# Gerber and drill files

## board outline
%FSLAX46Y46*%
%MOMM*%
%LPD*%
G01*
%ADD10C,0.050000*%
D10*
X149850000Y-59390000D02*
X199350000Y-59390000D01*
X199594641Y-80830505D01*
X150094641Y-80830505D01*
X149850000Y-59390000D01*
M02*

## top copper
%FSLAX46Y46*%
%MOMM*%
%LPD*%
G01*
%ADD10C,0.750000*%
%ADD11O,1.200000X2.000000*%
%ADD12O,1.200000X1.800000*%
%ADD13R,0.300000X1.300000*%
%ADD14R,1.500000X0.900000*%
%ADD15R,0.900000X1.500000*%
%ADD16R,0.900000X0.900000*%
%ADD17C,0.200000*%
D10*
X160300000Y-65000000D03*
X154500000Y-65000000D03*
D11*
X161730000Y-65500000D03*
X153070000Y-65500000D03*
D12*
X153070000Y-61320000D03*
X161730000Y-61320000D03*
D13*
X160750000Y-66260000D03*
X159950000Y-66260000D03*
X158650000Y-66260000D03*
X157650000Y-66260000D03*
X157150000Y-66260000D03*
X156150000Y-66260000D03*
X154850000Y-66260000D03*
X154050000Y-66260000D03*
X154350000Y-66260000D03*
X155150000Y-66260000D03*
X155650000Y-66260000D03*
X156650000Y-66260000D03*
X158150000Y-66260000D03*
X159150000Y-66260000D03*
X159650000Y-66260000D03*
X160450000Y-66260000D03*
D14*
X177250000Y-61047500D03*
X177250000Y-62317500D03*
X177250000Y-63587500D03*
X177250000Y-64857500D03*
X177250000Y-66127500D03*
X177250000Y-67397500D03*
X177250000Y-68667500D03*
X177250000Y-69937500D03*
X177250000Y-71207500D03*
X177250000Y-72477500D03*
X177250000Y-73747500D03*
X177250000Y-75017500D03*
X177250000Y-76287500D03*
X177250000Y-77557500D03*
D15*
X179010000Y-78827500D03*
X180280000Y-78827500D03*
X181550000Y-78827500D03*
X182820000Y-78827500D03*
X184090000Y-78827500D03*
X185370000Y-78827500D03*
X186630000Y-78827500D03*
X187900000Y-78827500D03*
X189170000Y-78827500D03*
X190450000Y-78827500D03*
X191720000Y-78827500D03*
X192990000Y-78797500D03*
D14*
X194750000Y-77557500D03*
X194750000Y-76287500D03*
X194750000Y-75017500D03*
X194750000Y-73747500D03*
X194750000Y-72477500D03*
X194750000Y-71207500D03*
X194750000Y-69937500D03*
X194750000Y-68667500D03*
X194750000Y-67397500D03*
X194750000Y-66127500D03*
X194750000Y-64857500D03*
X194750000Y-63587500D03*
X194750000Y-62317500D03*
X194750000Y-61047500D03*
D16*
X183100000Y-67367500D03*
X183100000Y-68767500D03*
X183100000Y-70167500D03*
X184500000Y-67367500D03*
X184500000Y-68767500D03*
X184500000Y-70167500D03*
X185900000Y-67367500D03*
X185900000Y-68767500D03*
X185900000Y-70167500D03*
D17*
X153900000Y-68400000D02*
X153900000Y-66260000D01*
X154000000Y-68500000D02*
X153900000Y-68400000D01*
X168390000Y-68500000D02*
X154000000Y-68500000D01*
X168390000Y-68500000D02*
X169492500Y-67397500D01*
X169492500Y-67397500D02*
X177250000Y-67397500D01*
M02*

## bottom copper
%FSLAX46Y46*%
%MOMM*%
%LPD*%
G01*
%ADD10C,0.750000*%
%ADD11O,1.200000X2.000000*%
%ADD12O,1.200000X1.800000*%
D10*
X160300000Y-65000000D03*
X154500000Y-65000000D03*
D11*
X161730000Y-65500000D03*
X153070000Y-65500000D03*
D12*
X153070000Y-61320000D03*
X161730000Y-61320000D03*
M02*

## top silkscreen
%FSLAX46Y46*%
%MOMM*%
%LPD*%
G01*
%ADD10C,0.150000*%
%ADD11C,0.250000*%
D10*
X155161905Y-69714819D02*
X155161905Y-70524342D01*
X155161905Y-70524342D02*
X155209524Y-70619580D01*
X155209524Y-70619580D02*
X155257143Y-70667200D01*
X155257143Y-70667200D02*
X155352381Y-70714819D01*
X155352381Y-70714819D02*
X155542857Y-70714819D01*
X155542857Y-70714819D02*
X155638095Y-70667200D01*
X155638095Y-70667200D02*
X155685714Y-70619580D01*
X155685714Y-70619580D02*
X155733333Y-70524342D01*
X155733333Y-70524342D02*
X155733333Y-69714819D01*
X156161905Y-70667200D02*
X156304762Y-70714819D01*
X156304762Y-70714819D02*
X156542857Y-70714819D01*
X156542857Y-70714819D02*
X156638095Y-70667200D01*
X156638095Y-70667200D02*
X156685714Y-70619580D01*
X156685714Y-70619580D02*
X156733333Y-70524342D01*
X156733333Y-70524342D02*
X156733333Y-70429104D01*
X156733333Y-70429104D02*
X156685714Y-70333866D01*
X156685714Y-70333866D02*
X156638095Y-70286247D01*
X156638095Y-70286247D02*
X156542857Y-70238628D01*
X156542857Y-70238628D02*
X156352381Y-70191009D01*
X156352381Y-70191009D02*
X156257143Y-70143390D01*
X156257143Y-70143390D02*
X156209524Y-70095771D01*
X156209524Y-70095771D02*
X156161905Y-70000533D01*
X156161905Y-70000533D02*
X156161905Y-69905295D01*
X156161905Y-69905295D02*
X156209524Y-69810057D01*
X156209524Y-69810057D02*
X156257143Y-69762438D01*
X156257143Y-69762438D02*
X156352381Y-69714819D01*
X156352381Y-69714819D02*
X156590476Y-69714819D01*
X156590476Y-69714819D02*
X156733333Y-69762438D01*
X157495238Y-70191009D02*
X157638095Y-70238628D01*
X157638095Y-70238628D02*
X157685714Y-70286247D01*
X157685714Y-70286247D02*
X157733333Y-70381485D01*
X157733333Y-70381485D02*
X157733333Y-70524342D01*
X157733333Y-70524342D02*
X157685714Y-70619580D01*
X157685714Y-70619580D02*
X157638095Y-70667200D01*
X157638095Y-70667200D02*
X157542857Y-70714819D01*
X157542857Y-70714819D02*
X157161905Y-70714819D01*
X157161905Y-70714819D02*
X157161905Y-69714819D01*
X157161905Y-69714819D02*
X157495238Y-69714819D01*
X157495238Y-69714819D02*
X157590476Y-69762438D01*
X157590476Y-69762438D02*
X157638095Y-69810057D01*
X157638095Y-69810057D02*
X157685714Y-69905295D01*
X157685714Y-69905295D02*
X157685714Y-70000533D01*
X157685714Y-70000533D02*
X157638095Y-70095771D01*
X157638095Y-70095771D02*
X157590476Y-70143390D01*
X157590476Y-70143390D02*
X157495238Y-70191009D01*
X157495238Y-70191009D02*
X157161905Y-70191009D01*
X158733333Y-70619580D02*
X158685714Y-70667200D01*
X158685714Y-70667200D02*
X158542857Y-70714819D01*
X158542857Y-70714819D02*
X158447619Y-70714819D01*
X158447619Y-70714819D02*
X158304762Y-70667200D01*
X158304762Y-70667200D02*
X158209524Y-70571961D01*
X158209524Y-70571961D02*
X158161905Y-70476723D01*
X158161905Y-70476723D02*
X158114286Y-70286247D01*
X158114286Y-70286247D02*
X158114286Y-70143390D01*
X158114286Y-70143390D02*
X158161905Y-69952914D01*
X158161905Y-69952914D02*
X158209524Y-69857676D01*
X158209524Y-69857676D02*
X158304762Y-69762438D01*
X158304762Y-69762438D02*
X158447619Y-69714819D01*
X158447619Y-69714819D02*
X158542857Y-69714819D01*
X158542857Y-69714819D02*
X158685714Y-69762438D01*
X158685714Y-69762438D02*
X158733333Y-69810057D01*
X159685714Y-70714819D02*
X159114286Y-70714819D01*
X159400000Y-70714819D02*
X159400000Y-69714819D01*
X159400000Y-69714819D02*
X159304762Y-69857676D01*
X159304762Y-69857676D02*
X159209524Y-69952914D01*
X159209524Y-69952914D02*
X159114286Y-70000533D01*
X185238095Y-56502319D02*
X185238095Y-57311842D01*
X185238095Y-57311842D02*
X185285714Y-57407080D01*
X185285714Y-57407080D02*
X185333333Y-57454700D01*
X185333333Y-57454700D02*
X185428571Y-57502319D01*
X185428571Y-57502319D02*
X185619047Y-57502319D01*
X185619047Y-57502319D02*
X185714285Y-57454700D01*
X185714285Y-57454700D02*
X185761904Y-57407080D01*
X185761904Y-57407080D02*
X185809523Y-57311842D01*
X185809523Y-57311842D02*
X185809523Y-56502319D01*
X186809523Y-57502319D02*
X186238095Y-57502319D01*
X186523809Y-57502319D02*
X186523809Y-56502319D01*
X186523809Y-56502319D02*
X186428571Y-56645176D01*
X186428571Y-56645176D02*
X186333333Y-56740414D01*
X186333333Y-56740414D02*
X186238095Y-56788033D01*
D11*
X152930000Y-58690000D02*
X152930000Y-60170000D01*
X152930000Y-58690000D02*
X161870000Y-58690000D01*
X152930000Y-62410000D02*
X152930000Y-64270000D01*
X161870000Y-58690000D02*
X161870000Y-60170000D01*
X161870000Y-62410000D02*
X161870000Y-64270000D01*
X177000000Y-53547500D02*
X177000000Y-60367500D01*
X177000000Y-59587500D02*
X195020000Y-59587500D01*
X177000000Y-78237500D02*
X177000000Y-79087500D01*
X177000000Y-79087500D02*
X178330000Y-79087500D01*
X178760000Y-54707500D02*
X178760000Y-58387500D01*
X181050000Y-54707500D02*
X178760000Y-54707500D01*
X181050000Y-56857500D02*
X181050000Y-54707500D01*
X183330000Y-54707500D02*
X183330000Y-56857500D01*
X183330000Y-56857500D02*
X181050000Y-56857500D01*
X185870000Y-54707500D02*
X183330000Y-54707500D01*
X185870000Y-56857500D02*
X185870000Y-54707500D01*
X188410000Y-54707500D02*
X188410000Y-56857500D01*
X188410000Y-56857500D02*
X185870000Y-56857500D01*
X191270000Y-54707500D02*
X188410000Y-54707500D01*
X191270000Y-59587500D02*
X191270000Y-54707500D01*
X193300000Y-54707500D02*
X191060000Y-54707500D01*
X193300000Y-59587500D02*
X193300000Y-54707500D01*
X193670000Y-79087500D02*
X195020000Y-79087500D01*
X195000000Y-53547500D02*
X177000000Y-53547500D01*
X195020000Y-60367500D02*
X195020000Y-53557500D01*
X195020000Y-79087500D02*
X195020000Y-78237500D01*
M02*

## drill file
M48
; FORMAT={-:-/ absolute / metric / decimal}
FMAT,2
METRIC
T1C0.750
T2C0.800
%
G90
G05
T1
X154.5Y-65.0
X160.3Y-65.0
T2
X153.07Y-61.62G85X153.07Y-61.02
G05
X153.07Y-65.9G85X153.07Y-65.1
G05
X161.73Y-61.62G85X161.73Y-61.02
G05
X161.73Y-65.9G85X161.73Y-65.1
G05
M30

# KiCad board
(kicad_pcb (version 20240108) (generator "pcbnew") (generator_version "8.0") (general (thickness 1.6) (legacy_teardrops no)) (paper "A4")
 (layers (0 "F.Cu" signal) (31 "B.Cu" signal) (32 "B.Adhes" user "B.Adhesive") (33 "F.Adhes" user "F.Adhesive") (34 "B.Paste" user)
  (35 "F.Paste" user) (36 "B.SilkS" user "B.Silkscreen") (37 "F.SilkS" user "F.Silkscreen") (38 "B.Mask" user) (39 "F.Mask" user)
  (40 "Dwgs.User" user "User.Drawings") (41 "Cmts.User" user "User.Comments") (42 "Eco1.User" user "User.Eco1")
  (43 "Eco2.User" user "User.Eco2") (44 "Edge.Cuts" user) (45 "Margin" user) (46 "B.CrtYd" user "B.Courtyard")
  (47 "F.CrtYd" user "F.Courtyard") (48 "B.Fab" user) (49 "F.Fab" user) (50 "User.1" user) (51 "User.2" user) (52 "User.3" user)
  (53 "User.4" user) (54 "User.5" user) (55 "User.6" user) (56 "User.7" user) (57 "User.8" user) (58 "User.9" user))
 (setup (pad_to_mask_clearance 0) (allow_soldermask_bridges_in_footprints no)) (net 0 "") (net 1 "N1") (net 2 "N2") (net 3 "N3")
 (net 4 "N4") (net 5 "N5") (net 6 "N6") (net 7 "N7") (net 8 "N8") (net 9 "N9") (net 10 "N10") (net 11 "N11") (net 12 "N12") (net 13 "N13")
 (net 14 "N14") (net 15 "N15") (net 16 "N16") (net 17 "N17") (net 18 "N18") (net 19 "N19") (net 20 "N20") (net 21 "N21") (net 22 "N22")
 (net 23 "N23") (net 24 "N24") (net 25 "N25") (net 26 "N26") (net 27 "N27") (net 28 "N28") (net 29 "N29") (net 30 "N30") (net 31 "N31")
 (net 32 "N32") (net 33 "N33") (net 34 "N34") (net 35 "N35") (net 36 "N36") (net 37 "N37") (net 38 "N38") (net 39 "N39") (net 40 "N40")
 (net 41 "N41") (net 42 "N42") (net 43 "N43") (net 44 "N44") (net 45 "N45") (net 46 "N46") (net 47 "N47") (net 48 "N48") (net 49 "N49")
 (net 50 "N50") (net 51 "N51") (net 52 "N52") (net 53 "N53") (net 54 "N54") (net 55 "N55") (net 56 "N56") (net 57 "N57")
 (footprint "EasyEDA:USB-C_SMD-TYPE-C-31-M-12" (layer "F.Cu") (at 157.4 63.79 180)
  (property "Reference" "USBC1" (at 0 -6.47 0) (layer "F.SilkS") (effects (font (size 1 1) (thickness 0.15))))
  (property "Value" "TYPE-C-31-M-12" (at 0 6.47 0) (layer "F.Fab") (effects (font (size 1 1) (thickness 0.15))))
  (fp_line (start 4.47 5.1) (end 4.47 3.62) (stroke (width 0.25) (type solid)) (layer "F.SilkS"))
  (fp_line (start 4.47 5.1) (end -4.47 5.1) (stroke (width 0.25) (type solid)) (layer "F.SilkS"))
  (fp_line (start 4.47 1.38) (end 4.47 -0.48) (stroke (width 0.25) (type solid)) (layer "F.SilkS"))
  (fp_line (start -4.47 5.1) (end -4.47 3.62) (stroke (width 0.25) (type solid)) (layer "F.SilkS"))
  (fp_line (start -4.47 1.38) (end -4.47 -0.48) (stroke (width 0.25) (type solid)) (layer "F.SilkS"))
  (pad "" thru_hole circle (at -2.9 -1.21 180) (size 0.75 0.75) (drill 0.75) (layers "*.Cu" "*.Mask") (remove_unused_layers no))
  (pad "" thru_hole circle (at 2.9 -1.21 180) (size 0.75 0.75) (drill 0.75) (layers "*.Cu" "*.Mask") (remove_unused_layers no))
  (pad "0" thru_hole oval (at -4.33 -1.71 180) (size 1.2 2) (drill oval 0.799998 1.600022) (layers "*.Cu" "*.Mask")
   (remove_unused_layers no) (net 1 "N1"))
  (pad "1" thru_hole oval (at 4.33 -1.71 180) (size 1.2 2) (drill oval 0.799998 1.599971) (layers "*.Cu" "*.Mask") (remove_unused_layers no))
  (pad "2" thru_hole oval (at 4.33 2.47 180) (size 1.2 1.8) (drill oval 0.799998 1.399997) (layers "*.Cu" "*.Mask")
   (remove_unused_layers no))
  (pad "3" thru_hole oval (at -4.33 2.47 180) (size 1.2 1.8) (drill oval 0.799998 1.399997) (layers "*.Cu" "*.Mask")
   (remove_unused_layers no))
  (pad "A1" smd rect (at -3.35 -2.47 180) (size 0.3 1.3) (layers "F.Cu" "F.Paste" "F.Mask") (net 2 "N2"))
  (pad "A4" smd rect (at -2.55 -2.47 180) (size 0.3 1.3) (layers "F.Cu" "F.Paste" "F.Mask") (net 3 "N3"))
  (pad "A5" smd rect (at -1.25 -2.47 180) (size 0.3 1.3) (layers "F.Cu" "F.Paste" "F.Mask") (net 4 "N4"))
  (pad "A6" smd rect (at -0.25 -2.47 180) (size 0.3 1.3) (layers "F.Cu" "F.Paste" "F.Mask") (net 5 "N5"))
  (pad "A7" smd rect (at 0.25 -2.47 180) (size 0.3 1.3) (layers "F.Cu" "F.Paste" "F.Mask") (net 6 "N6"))
  (pad "A8" smd rect (at 1.25 -2.47 180) (size 0.3 1.3) (layers "F.Cu" "F.Paste" "F.Mask") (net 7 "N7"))
  (pad "A9" smd rect (at 2.55 -2.47 180) (size 0.3 1.3) (layers "F.Cu" "F.Paste" "F.Mask") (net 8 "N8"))
  (pad "A12" smd rect (at 3.35 -2.47 180) (size 0.3 1.3) (layers "F.Cu" "F.Paste" "F.Mask") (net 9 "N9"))
  (pad "B1" smd rect (at 3.05 -2.47 180) (size 0.3 1.3) (layers "F.Cu" "F.Paste" "F.Mask") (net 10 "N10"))
  (pad "B4" smd rect (at 2.25 -2.47 180) (size 0.3 1.3) (layers "F.Cu" "F.Paste" "F.Mask") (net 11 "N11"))
  (pad "B5" smd rect (at 1.75 -2.47 180) (size 0.3 1.3) (layers "F.Cu" "F.Paste" "F.Mask") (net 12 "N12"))
  (pad "B6" smd rect (at 0.75 -2.47 180) (size 0.3 1.3) (layers "F.Cu" "F.Paste" "F.Mask") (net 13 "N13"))
  (pad "B7" smd rect (at -0.75 -2.47 180) (size 0.3 1.3) (layers "F.Cu" "F.Paste" "F.Mask") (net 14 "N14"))
  (pad "B8" smd rect (at -1.75 -2.47 180) (size 0.3 1.3) (layers "F.Cu" "F.Paste" "F.Mask") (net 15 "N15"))
  (pad "B9" smd rect (at -2.25 -2.47 180) (size 0.3 1.3) (layers "F.Cu" "F.Paste" "F.Mask") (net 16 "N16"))
  (pad "B12" smd rect (at -3.05 -2.47 180) (size 0.3 1.3) (layers "F.Cu" "F.Paste" "F.Mask") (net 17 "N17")))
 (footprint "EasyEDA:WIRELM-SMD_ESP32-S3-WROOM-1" (layer "F.Cu") (at 186 69.9375)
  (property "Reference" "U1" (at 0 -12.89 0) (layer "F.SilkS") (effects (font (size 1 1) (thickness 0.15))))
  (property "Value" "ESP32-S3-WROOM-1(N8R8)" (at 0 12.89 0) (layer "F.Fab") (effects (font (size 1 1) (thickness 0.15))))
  (fp_line (start -9 -16.39) (end -9 -9.57) (stroke (width 0.25) (type solid)) (layer "F.SilkS"))
  (fp_line (start -9 -10.35) (end 9.02 -10.35) (stroke (width 0.25) (type solid)) (layer "F.SilkS"))
  (fp_line (start -9 8.3) (end -9 9.15) (stroke (width 0.25) (type solid)) (layer "F.SilkS"))
  (fp_line (start -9 9.15) (end -7.67 9.15) (stroke (width 0.25) (type solid)) (layer "F.SilkS"))
  (fp_line (start -7.24 -15.23) (end -7.24 -11.55) (stroke (width 0.25) (type solid)) (layer "F.SilkS"))
  (fp_line (start -4.95 -15.23) (end -7.24 -15.23) (stroke (width 0.25) (type solid)) (layer "F.SilkS"))
  (fp_line (start -4.95 -13.08) (end -4.95 -15.23) (stroke (width 0.25) (type solid)) (layer "F.SilkS"))
  (fp_line (start -2.67 -15.23) (end -2.67 -13.08) (stroke (width 0.25) (type solid)) (layer "F.SilkS"))
  (fp_line (start -2.67 -13.08) (end -4.95 -13.08) (stroke (width 0.25) (type solid)) (layer "F.SilkS"))
  (fp_line (start -0.13 -15.23) (end -2.67 -15.23) (stroke (width 0.25) (type solid)) (layer "F.SilkS"))
  (fp_line (start -0.13 -13.08) (end -0.13 -15.23) (stroke (width 0.25) (type solid)) (layer "F.SilkS"))
  (fp_line (start 2.41 -15.23) (end 2.41 -13.08) (stroke (width 0.25) (type solid)) (layer "F.SilkS"))
  (fp_line (start 2.41 -13.08) (end -0.13 -13.08) (stroke (width 0.25) (type solid)) (layer "F.SilkS"))
  (fp_line (start 5.27 -15.23) (end 2.41 -15.23) (stroke (width 0.25) (type solid)) (layer "F.SilkS"))
  (fp_line (start 5.27 -10.35) (end 5.27 -15.23) (stroke (width 0.25) (type solid)) (layer "F.SilkS"))
  (fp_line (start 7.3 -15.23) (end 5.06 -15.23) (stroke (width 0.25) (type solid)) (layer "F.SilkS"))
  (fp_line (start 7.3 -10.35) (end 7.3 -15.23) (stroke (width 0.25) (type solid)) (layer "F.SilkS"))
  (fp_line (start 7.67 9.15) (end 9.02 9.15) (stroke (width 0.25) (type solid)) (layer "F.SilkS"))
  (fp_line (start 9 -16.39) (end -9 -16.39) (stroke (width 0.25) (type solid)) (layer "F.SilkS"))
  (fp_line (start 9.02 -9.57) (end 9.02 -16.38) (stroke (width 0.25) (type solid)) (layer "F.SilkS"))
  (fp_line (start 9.02 9.15) (end 9.02 8.3) (stroke (width 0.25) (type solid)) (layer "F.SilkS"))
  (pad "1" smd rect (at -8.75 -8.89) (size 1.5 0.9) (layers "F.Cu" "F.Paste" "F.Mask") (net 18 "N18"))
  (pad "2" smd rect (at -8.75 -7.62) (size 1.5 0.9) (layers "F.Cu" "F.Paste" "F.Mask") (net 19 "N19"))
  (pad "3" smd rect (at -8.75 -6.35) (size 1.5 0.9) (layers "F.Cu" "F.Paste" "F.Mask") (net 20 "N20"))
  (pad "4" smd rect (at -8.75 -5.08) (size 1.5 0.9) (layers "F.Cu" "F.Paste" "F.Mask") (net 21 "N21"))
  (pad "5" smd rect (at -8.75 -3.81) (size 1.5 0.9) (layers "F.Cu" "F.Paste" "F.Mask") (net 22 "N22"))
  (pad "6" smd rect (at -8.75 -2.54) (size 1.5 0.9) (layers "F.Cu" "F.Paste" "F.Mask") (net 9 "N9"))
  (pad "7" smd rect (at -8.75 -1.27) (size 1.5 0.9) (layers "F.Cu" "F.Paste" "F.Mask") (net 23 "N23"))
  (pad "8" smd rect (at -8.75 0) (size 1.5 0.9) (layers "F.Cu" "F.Paste" "F.Mask") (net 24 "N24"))
  (pad "9" smd rect (at -8.75 1.27) (size 1.5 0.9) (layers "F.Cu" "F.Paste" "F.Mask") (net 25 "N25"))
  (pad "10" smd rect (at -8.75 2.54) (size 1.5 0.9) (layers "F.Cu" "F.Paste" "F.Mask") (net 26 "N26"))
  (pad "11" smd rect (at -8.75 3.81) (size 1.5 0.9) (layers "F.Cu" "F.Paste" "F.Mask") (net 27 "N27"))
  (pad "12" smd rect (at -8.75 5.08) (size 1.5 0.9) (layers "F.Cu" "F.Paste" "F.Mask") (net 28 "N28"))
  (pad "13" smd rect (at -8.75 6.35) (size 1.5 0.9) (layers "F.Cu" "F.Paste" "F.Mask") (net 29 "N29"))
  (pad "14" smd rect (at -8.75 7.62) (size 1.5 0.9) (layers "F.Cu" "F.Paste" "F.Mask") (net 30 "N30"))
  (pad "15" smd rect (at -6.99 8.89 90) (size 1.5 0.9) (layers "F.Cu" "F.Paste" "F.Mask") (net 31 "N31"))
  (pad "16" smd rect (at -5.72 8.89 90) (size 1.5 0.9) (layers "F.Cu" "F.Paste" "F.Mask") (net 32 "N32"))
  (pad "17" smd rect (at -4.45 8.89 90) (size 1.5 0.9) (layers "F.Cu" "F.Paste" "F.Mask") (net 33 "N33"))
  (pad "18" smd rect (at -3.18 8.89 90) (size 1.5 0.9) (layers "F.Cu" "F.Paste" "F.Mask") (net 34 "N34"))
  (pad "19" smd rect (at -1.91 8.89 90) (size 1.5 0.9) (layers "F.Cu" "F.Paste" "F.Mask") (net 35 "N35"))
  (pad "20" smd rect (at -0.63 8.89 90) (size 1.5 0.9) (layers "F.Cu" "F.Paste" "F.Mask") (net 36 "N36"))
  (pad "21" smd rect (at 0.63 8.89 90) (size 1.5 0.9) (layers "F.Cu" "F.Paste" "F.Mask") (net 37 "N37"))
  (pad "22" smd rect (at 1.9 8.89 90) (size 1.5 0.9) (layers "F.Cu" "F.Paste" "F.Mask") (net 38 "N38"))
  (pad "23" smd rect (at 3.17 8.89 90) (size 1.5 0.9) (layers "F.Cu" "F.Paste" "F.Mask") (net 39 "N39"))
  (pad "24" smd rect (at 4.45 8.89 90) (size 1.5 0.9) (layers "F.Cu" "F.Paste" "F.Mask") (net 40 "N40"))
  (pad "25" smd rect (at 5.72 8.89 90) (size 1.5 0.9) (layers "F.Cu" "F.Paste" "F.Mask") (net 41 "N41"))
  (pad "26" smd rect (at 6.99 8.86 90) (size 1.5 0.9) (layers "F.Cu" "F.Paste" "F.Mask") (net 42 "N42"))
  (pad "27" smd rect (at 8.75 7.62 180) (size 1.5 0.9) (layers "F.Cu" "F.Paste" "F.Mask") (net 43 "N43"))
  (pad "28" smd rect (at 8.75 6.35 180) (size 1.5 0.9) (layers "F.Cu" "F.Paste" "F.Mask") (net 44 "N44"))
  (pad "29" smd rect (at 8.75 5.08 180) (size 1.5 0.9) (layers "F.Cu" "F.Paste" "F.Mask") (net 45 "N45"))
  (pad "30" smd rect (at 8.75 3.81 180) (size 1.5 0.9) (layers "F.Cu" "F.Paste" "F.Mask") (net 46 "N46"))
  (pad "31" smd rect (at 8.75 2.54 180) (size 1.5 0.9) (layers "F.Cu" "F.Paste" "F.Mask") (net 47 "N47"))
  (pad "32" smd rect (at 8.75 1.27 180) (size 1.5 0.9) (layers "F.Cu" "F.Paste" "F.Mask") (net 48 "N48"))
  (pad "33" smd rect (at 8.75 0 180) (size 1.5 0.9) (layers "F.Cu" "F.Paste" "F.Mask") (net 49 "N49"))
  (pad "34" smd rect (at 8.75 -1.27 180) (size 1.5 0.9) (layers "F.Cu" "F.Paste" "F.Mask") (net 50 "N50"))
  (pad "35" smd rect (at 8.75 -2.54 180) (size 1.5 0.9) (layers "F.Cu" "F.Paste" "F.Mask") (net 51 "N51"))
  (pad "36" smd rect (at 8.75 -3.81 180) (size 1.5 0.9) (layers "F.Cu" "F.Paste" "F.Mask") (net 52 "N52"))
  (pad "37" smd rect (at 8.75 -5.08 180) (size 1.5 0.9) (layers "F.Cu" "F.Paste" "F.Mask") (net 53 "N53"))
  (pad "38" smd rect (at 8.75 -6.35 180) (size 1.5 0.9) (layers "F.Cu" "F.Paste" "F.Mask") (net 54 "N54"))
  (pad "39" smd rect (at 8.75 -7.62 180) (size 1.5 0.9) (layers "F.Cu" "F.Paste" "F.Mask") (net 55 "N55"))
  (pad "40" smd rect (at 8.75 -8.89 180) (size 1.5 0.9) (layers "F.Cu" "F.Paste" "F.Mask") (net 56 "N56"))
  (pad "41" smd rect (at -2.9 -2.57 90) (size 0.9 0.9) (layers "F.Cu" "F.Paste" "F.Mask") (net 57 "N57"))
  (pad "41" smd rect (at -2.9 -1.17 90) (size 0.9 0.9) (layers "F.Cu" "F.Paste" "F.Mask") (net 57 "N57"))
  (pad "41" smd rect (at -2.9 0.23 90) (size 0.9 0.9) (layers "F.Cu" "F.Paste" "F.Mask") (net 57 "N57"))
  (pad "41" smd rect (at -1.5 -2.57 90) (size 0.9 0.9) (layers "F.Cu" "F.Paste" "F.Mask") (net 57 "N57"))
  (pad "41" smd rect (at -1.5 -1.17 90) (size 0.9 0.9) (layers "F.Cu" "F.Paste" "F.Mask") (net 57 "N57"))
  (pad "41" smd rect (at -1.5 0.23 90) (size 0.9 0.9) (layers "F.Cu" "F.Paste" "F.Mask") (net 57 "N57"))
  (pad "41" smd rect (at -0.1 -2.57 90) (size 0.9 0.9) (layers "F.Cu" "F.Paste" "F.Mask") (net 57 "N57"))
  (pad "41" smd rect (at -0.1 -1.17 90) (size 0.9 0.9) (layers "F.Cu" "F.Paste" "F.Mask") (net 57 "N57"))
  (pad "41" smd rect (at -0.1 0.23 90) (size 0.9 0.9) (layers "F.Cu" "F.Paste" "F.Mask") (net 57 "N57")))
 (gr_poly
  (pts (xy 149.85 59.39) (xy 199.35 59.39) (xy 199.594641 80.830505) (xy 150.094641 80.830505)) (stroke (width 0.05) (type solid))
  (fill none) (layer "Edge.Cuts"))
 (segment (start 153.9 68.4) (end 153.9 66.26) (width 0.2) (layer "F.Cu") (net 9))
 (segment (start 154 68.5) (end 153.9 68.4) (width 0.2) (layer "F.Cu") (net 9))
 (segment (start 168.39 68.5) (end 154 68.5) (width 0.2) (layer "F.Cu") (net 9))
 (segment (start 168.39 68.5) (end 169.4925 67.3975) (width 0.2) (layer "F.Cu") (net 9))
 (segment (start 169.4925 67.3975) (end 177.25 67.3975) (width 0.2) (layer "F.Cu") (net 9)))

